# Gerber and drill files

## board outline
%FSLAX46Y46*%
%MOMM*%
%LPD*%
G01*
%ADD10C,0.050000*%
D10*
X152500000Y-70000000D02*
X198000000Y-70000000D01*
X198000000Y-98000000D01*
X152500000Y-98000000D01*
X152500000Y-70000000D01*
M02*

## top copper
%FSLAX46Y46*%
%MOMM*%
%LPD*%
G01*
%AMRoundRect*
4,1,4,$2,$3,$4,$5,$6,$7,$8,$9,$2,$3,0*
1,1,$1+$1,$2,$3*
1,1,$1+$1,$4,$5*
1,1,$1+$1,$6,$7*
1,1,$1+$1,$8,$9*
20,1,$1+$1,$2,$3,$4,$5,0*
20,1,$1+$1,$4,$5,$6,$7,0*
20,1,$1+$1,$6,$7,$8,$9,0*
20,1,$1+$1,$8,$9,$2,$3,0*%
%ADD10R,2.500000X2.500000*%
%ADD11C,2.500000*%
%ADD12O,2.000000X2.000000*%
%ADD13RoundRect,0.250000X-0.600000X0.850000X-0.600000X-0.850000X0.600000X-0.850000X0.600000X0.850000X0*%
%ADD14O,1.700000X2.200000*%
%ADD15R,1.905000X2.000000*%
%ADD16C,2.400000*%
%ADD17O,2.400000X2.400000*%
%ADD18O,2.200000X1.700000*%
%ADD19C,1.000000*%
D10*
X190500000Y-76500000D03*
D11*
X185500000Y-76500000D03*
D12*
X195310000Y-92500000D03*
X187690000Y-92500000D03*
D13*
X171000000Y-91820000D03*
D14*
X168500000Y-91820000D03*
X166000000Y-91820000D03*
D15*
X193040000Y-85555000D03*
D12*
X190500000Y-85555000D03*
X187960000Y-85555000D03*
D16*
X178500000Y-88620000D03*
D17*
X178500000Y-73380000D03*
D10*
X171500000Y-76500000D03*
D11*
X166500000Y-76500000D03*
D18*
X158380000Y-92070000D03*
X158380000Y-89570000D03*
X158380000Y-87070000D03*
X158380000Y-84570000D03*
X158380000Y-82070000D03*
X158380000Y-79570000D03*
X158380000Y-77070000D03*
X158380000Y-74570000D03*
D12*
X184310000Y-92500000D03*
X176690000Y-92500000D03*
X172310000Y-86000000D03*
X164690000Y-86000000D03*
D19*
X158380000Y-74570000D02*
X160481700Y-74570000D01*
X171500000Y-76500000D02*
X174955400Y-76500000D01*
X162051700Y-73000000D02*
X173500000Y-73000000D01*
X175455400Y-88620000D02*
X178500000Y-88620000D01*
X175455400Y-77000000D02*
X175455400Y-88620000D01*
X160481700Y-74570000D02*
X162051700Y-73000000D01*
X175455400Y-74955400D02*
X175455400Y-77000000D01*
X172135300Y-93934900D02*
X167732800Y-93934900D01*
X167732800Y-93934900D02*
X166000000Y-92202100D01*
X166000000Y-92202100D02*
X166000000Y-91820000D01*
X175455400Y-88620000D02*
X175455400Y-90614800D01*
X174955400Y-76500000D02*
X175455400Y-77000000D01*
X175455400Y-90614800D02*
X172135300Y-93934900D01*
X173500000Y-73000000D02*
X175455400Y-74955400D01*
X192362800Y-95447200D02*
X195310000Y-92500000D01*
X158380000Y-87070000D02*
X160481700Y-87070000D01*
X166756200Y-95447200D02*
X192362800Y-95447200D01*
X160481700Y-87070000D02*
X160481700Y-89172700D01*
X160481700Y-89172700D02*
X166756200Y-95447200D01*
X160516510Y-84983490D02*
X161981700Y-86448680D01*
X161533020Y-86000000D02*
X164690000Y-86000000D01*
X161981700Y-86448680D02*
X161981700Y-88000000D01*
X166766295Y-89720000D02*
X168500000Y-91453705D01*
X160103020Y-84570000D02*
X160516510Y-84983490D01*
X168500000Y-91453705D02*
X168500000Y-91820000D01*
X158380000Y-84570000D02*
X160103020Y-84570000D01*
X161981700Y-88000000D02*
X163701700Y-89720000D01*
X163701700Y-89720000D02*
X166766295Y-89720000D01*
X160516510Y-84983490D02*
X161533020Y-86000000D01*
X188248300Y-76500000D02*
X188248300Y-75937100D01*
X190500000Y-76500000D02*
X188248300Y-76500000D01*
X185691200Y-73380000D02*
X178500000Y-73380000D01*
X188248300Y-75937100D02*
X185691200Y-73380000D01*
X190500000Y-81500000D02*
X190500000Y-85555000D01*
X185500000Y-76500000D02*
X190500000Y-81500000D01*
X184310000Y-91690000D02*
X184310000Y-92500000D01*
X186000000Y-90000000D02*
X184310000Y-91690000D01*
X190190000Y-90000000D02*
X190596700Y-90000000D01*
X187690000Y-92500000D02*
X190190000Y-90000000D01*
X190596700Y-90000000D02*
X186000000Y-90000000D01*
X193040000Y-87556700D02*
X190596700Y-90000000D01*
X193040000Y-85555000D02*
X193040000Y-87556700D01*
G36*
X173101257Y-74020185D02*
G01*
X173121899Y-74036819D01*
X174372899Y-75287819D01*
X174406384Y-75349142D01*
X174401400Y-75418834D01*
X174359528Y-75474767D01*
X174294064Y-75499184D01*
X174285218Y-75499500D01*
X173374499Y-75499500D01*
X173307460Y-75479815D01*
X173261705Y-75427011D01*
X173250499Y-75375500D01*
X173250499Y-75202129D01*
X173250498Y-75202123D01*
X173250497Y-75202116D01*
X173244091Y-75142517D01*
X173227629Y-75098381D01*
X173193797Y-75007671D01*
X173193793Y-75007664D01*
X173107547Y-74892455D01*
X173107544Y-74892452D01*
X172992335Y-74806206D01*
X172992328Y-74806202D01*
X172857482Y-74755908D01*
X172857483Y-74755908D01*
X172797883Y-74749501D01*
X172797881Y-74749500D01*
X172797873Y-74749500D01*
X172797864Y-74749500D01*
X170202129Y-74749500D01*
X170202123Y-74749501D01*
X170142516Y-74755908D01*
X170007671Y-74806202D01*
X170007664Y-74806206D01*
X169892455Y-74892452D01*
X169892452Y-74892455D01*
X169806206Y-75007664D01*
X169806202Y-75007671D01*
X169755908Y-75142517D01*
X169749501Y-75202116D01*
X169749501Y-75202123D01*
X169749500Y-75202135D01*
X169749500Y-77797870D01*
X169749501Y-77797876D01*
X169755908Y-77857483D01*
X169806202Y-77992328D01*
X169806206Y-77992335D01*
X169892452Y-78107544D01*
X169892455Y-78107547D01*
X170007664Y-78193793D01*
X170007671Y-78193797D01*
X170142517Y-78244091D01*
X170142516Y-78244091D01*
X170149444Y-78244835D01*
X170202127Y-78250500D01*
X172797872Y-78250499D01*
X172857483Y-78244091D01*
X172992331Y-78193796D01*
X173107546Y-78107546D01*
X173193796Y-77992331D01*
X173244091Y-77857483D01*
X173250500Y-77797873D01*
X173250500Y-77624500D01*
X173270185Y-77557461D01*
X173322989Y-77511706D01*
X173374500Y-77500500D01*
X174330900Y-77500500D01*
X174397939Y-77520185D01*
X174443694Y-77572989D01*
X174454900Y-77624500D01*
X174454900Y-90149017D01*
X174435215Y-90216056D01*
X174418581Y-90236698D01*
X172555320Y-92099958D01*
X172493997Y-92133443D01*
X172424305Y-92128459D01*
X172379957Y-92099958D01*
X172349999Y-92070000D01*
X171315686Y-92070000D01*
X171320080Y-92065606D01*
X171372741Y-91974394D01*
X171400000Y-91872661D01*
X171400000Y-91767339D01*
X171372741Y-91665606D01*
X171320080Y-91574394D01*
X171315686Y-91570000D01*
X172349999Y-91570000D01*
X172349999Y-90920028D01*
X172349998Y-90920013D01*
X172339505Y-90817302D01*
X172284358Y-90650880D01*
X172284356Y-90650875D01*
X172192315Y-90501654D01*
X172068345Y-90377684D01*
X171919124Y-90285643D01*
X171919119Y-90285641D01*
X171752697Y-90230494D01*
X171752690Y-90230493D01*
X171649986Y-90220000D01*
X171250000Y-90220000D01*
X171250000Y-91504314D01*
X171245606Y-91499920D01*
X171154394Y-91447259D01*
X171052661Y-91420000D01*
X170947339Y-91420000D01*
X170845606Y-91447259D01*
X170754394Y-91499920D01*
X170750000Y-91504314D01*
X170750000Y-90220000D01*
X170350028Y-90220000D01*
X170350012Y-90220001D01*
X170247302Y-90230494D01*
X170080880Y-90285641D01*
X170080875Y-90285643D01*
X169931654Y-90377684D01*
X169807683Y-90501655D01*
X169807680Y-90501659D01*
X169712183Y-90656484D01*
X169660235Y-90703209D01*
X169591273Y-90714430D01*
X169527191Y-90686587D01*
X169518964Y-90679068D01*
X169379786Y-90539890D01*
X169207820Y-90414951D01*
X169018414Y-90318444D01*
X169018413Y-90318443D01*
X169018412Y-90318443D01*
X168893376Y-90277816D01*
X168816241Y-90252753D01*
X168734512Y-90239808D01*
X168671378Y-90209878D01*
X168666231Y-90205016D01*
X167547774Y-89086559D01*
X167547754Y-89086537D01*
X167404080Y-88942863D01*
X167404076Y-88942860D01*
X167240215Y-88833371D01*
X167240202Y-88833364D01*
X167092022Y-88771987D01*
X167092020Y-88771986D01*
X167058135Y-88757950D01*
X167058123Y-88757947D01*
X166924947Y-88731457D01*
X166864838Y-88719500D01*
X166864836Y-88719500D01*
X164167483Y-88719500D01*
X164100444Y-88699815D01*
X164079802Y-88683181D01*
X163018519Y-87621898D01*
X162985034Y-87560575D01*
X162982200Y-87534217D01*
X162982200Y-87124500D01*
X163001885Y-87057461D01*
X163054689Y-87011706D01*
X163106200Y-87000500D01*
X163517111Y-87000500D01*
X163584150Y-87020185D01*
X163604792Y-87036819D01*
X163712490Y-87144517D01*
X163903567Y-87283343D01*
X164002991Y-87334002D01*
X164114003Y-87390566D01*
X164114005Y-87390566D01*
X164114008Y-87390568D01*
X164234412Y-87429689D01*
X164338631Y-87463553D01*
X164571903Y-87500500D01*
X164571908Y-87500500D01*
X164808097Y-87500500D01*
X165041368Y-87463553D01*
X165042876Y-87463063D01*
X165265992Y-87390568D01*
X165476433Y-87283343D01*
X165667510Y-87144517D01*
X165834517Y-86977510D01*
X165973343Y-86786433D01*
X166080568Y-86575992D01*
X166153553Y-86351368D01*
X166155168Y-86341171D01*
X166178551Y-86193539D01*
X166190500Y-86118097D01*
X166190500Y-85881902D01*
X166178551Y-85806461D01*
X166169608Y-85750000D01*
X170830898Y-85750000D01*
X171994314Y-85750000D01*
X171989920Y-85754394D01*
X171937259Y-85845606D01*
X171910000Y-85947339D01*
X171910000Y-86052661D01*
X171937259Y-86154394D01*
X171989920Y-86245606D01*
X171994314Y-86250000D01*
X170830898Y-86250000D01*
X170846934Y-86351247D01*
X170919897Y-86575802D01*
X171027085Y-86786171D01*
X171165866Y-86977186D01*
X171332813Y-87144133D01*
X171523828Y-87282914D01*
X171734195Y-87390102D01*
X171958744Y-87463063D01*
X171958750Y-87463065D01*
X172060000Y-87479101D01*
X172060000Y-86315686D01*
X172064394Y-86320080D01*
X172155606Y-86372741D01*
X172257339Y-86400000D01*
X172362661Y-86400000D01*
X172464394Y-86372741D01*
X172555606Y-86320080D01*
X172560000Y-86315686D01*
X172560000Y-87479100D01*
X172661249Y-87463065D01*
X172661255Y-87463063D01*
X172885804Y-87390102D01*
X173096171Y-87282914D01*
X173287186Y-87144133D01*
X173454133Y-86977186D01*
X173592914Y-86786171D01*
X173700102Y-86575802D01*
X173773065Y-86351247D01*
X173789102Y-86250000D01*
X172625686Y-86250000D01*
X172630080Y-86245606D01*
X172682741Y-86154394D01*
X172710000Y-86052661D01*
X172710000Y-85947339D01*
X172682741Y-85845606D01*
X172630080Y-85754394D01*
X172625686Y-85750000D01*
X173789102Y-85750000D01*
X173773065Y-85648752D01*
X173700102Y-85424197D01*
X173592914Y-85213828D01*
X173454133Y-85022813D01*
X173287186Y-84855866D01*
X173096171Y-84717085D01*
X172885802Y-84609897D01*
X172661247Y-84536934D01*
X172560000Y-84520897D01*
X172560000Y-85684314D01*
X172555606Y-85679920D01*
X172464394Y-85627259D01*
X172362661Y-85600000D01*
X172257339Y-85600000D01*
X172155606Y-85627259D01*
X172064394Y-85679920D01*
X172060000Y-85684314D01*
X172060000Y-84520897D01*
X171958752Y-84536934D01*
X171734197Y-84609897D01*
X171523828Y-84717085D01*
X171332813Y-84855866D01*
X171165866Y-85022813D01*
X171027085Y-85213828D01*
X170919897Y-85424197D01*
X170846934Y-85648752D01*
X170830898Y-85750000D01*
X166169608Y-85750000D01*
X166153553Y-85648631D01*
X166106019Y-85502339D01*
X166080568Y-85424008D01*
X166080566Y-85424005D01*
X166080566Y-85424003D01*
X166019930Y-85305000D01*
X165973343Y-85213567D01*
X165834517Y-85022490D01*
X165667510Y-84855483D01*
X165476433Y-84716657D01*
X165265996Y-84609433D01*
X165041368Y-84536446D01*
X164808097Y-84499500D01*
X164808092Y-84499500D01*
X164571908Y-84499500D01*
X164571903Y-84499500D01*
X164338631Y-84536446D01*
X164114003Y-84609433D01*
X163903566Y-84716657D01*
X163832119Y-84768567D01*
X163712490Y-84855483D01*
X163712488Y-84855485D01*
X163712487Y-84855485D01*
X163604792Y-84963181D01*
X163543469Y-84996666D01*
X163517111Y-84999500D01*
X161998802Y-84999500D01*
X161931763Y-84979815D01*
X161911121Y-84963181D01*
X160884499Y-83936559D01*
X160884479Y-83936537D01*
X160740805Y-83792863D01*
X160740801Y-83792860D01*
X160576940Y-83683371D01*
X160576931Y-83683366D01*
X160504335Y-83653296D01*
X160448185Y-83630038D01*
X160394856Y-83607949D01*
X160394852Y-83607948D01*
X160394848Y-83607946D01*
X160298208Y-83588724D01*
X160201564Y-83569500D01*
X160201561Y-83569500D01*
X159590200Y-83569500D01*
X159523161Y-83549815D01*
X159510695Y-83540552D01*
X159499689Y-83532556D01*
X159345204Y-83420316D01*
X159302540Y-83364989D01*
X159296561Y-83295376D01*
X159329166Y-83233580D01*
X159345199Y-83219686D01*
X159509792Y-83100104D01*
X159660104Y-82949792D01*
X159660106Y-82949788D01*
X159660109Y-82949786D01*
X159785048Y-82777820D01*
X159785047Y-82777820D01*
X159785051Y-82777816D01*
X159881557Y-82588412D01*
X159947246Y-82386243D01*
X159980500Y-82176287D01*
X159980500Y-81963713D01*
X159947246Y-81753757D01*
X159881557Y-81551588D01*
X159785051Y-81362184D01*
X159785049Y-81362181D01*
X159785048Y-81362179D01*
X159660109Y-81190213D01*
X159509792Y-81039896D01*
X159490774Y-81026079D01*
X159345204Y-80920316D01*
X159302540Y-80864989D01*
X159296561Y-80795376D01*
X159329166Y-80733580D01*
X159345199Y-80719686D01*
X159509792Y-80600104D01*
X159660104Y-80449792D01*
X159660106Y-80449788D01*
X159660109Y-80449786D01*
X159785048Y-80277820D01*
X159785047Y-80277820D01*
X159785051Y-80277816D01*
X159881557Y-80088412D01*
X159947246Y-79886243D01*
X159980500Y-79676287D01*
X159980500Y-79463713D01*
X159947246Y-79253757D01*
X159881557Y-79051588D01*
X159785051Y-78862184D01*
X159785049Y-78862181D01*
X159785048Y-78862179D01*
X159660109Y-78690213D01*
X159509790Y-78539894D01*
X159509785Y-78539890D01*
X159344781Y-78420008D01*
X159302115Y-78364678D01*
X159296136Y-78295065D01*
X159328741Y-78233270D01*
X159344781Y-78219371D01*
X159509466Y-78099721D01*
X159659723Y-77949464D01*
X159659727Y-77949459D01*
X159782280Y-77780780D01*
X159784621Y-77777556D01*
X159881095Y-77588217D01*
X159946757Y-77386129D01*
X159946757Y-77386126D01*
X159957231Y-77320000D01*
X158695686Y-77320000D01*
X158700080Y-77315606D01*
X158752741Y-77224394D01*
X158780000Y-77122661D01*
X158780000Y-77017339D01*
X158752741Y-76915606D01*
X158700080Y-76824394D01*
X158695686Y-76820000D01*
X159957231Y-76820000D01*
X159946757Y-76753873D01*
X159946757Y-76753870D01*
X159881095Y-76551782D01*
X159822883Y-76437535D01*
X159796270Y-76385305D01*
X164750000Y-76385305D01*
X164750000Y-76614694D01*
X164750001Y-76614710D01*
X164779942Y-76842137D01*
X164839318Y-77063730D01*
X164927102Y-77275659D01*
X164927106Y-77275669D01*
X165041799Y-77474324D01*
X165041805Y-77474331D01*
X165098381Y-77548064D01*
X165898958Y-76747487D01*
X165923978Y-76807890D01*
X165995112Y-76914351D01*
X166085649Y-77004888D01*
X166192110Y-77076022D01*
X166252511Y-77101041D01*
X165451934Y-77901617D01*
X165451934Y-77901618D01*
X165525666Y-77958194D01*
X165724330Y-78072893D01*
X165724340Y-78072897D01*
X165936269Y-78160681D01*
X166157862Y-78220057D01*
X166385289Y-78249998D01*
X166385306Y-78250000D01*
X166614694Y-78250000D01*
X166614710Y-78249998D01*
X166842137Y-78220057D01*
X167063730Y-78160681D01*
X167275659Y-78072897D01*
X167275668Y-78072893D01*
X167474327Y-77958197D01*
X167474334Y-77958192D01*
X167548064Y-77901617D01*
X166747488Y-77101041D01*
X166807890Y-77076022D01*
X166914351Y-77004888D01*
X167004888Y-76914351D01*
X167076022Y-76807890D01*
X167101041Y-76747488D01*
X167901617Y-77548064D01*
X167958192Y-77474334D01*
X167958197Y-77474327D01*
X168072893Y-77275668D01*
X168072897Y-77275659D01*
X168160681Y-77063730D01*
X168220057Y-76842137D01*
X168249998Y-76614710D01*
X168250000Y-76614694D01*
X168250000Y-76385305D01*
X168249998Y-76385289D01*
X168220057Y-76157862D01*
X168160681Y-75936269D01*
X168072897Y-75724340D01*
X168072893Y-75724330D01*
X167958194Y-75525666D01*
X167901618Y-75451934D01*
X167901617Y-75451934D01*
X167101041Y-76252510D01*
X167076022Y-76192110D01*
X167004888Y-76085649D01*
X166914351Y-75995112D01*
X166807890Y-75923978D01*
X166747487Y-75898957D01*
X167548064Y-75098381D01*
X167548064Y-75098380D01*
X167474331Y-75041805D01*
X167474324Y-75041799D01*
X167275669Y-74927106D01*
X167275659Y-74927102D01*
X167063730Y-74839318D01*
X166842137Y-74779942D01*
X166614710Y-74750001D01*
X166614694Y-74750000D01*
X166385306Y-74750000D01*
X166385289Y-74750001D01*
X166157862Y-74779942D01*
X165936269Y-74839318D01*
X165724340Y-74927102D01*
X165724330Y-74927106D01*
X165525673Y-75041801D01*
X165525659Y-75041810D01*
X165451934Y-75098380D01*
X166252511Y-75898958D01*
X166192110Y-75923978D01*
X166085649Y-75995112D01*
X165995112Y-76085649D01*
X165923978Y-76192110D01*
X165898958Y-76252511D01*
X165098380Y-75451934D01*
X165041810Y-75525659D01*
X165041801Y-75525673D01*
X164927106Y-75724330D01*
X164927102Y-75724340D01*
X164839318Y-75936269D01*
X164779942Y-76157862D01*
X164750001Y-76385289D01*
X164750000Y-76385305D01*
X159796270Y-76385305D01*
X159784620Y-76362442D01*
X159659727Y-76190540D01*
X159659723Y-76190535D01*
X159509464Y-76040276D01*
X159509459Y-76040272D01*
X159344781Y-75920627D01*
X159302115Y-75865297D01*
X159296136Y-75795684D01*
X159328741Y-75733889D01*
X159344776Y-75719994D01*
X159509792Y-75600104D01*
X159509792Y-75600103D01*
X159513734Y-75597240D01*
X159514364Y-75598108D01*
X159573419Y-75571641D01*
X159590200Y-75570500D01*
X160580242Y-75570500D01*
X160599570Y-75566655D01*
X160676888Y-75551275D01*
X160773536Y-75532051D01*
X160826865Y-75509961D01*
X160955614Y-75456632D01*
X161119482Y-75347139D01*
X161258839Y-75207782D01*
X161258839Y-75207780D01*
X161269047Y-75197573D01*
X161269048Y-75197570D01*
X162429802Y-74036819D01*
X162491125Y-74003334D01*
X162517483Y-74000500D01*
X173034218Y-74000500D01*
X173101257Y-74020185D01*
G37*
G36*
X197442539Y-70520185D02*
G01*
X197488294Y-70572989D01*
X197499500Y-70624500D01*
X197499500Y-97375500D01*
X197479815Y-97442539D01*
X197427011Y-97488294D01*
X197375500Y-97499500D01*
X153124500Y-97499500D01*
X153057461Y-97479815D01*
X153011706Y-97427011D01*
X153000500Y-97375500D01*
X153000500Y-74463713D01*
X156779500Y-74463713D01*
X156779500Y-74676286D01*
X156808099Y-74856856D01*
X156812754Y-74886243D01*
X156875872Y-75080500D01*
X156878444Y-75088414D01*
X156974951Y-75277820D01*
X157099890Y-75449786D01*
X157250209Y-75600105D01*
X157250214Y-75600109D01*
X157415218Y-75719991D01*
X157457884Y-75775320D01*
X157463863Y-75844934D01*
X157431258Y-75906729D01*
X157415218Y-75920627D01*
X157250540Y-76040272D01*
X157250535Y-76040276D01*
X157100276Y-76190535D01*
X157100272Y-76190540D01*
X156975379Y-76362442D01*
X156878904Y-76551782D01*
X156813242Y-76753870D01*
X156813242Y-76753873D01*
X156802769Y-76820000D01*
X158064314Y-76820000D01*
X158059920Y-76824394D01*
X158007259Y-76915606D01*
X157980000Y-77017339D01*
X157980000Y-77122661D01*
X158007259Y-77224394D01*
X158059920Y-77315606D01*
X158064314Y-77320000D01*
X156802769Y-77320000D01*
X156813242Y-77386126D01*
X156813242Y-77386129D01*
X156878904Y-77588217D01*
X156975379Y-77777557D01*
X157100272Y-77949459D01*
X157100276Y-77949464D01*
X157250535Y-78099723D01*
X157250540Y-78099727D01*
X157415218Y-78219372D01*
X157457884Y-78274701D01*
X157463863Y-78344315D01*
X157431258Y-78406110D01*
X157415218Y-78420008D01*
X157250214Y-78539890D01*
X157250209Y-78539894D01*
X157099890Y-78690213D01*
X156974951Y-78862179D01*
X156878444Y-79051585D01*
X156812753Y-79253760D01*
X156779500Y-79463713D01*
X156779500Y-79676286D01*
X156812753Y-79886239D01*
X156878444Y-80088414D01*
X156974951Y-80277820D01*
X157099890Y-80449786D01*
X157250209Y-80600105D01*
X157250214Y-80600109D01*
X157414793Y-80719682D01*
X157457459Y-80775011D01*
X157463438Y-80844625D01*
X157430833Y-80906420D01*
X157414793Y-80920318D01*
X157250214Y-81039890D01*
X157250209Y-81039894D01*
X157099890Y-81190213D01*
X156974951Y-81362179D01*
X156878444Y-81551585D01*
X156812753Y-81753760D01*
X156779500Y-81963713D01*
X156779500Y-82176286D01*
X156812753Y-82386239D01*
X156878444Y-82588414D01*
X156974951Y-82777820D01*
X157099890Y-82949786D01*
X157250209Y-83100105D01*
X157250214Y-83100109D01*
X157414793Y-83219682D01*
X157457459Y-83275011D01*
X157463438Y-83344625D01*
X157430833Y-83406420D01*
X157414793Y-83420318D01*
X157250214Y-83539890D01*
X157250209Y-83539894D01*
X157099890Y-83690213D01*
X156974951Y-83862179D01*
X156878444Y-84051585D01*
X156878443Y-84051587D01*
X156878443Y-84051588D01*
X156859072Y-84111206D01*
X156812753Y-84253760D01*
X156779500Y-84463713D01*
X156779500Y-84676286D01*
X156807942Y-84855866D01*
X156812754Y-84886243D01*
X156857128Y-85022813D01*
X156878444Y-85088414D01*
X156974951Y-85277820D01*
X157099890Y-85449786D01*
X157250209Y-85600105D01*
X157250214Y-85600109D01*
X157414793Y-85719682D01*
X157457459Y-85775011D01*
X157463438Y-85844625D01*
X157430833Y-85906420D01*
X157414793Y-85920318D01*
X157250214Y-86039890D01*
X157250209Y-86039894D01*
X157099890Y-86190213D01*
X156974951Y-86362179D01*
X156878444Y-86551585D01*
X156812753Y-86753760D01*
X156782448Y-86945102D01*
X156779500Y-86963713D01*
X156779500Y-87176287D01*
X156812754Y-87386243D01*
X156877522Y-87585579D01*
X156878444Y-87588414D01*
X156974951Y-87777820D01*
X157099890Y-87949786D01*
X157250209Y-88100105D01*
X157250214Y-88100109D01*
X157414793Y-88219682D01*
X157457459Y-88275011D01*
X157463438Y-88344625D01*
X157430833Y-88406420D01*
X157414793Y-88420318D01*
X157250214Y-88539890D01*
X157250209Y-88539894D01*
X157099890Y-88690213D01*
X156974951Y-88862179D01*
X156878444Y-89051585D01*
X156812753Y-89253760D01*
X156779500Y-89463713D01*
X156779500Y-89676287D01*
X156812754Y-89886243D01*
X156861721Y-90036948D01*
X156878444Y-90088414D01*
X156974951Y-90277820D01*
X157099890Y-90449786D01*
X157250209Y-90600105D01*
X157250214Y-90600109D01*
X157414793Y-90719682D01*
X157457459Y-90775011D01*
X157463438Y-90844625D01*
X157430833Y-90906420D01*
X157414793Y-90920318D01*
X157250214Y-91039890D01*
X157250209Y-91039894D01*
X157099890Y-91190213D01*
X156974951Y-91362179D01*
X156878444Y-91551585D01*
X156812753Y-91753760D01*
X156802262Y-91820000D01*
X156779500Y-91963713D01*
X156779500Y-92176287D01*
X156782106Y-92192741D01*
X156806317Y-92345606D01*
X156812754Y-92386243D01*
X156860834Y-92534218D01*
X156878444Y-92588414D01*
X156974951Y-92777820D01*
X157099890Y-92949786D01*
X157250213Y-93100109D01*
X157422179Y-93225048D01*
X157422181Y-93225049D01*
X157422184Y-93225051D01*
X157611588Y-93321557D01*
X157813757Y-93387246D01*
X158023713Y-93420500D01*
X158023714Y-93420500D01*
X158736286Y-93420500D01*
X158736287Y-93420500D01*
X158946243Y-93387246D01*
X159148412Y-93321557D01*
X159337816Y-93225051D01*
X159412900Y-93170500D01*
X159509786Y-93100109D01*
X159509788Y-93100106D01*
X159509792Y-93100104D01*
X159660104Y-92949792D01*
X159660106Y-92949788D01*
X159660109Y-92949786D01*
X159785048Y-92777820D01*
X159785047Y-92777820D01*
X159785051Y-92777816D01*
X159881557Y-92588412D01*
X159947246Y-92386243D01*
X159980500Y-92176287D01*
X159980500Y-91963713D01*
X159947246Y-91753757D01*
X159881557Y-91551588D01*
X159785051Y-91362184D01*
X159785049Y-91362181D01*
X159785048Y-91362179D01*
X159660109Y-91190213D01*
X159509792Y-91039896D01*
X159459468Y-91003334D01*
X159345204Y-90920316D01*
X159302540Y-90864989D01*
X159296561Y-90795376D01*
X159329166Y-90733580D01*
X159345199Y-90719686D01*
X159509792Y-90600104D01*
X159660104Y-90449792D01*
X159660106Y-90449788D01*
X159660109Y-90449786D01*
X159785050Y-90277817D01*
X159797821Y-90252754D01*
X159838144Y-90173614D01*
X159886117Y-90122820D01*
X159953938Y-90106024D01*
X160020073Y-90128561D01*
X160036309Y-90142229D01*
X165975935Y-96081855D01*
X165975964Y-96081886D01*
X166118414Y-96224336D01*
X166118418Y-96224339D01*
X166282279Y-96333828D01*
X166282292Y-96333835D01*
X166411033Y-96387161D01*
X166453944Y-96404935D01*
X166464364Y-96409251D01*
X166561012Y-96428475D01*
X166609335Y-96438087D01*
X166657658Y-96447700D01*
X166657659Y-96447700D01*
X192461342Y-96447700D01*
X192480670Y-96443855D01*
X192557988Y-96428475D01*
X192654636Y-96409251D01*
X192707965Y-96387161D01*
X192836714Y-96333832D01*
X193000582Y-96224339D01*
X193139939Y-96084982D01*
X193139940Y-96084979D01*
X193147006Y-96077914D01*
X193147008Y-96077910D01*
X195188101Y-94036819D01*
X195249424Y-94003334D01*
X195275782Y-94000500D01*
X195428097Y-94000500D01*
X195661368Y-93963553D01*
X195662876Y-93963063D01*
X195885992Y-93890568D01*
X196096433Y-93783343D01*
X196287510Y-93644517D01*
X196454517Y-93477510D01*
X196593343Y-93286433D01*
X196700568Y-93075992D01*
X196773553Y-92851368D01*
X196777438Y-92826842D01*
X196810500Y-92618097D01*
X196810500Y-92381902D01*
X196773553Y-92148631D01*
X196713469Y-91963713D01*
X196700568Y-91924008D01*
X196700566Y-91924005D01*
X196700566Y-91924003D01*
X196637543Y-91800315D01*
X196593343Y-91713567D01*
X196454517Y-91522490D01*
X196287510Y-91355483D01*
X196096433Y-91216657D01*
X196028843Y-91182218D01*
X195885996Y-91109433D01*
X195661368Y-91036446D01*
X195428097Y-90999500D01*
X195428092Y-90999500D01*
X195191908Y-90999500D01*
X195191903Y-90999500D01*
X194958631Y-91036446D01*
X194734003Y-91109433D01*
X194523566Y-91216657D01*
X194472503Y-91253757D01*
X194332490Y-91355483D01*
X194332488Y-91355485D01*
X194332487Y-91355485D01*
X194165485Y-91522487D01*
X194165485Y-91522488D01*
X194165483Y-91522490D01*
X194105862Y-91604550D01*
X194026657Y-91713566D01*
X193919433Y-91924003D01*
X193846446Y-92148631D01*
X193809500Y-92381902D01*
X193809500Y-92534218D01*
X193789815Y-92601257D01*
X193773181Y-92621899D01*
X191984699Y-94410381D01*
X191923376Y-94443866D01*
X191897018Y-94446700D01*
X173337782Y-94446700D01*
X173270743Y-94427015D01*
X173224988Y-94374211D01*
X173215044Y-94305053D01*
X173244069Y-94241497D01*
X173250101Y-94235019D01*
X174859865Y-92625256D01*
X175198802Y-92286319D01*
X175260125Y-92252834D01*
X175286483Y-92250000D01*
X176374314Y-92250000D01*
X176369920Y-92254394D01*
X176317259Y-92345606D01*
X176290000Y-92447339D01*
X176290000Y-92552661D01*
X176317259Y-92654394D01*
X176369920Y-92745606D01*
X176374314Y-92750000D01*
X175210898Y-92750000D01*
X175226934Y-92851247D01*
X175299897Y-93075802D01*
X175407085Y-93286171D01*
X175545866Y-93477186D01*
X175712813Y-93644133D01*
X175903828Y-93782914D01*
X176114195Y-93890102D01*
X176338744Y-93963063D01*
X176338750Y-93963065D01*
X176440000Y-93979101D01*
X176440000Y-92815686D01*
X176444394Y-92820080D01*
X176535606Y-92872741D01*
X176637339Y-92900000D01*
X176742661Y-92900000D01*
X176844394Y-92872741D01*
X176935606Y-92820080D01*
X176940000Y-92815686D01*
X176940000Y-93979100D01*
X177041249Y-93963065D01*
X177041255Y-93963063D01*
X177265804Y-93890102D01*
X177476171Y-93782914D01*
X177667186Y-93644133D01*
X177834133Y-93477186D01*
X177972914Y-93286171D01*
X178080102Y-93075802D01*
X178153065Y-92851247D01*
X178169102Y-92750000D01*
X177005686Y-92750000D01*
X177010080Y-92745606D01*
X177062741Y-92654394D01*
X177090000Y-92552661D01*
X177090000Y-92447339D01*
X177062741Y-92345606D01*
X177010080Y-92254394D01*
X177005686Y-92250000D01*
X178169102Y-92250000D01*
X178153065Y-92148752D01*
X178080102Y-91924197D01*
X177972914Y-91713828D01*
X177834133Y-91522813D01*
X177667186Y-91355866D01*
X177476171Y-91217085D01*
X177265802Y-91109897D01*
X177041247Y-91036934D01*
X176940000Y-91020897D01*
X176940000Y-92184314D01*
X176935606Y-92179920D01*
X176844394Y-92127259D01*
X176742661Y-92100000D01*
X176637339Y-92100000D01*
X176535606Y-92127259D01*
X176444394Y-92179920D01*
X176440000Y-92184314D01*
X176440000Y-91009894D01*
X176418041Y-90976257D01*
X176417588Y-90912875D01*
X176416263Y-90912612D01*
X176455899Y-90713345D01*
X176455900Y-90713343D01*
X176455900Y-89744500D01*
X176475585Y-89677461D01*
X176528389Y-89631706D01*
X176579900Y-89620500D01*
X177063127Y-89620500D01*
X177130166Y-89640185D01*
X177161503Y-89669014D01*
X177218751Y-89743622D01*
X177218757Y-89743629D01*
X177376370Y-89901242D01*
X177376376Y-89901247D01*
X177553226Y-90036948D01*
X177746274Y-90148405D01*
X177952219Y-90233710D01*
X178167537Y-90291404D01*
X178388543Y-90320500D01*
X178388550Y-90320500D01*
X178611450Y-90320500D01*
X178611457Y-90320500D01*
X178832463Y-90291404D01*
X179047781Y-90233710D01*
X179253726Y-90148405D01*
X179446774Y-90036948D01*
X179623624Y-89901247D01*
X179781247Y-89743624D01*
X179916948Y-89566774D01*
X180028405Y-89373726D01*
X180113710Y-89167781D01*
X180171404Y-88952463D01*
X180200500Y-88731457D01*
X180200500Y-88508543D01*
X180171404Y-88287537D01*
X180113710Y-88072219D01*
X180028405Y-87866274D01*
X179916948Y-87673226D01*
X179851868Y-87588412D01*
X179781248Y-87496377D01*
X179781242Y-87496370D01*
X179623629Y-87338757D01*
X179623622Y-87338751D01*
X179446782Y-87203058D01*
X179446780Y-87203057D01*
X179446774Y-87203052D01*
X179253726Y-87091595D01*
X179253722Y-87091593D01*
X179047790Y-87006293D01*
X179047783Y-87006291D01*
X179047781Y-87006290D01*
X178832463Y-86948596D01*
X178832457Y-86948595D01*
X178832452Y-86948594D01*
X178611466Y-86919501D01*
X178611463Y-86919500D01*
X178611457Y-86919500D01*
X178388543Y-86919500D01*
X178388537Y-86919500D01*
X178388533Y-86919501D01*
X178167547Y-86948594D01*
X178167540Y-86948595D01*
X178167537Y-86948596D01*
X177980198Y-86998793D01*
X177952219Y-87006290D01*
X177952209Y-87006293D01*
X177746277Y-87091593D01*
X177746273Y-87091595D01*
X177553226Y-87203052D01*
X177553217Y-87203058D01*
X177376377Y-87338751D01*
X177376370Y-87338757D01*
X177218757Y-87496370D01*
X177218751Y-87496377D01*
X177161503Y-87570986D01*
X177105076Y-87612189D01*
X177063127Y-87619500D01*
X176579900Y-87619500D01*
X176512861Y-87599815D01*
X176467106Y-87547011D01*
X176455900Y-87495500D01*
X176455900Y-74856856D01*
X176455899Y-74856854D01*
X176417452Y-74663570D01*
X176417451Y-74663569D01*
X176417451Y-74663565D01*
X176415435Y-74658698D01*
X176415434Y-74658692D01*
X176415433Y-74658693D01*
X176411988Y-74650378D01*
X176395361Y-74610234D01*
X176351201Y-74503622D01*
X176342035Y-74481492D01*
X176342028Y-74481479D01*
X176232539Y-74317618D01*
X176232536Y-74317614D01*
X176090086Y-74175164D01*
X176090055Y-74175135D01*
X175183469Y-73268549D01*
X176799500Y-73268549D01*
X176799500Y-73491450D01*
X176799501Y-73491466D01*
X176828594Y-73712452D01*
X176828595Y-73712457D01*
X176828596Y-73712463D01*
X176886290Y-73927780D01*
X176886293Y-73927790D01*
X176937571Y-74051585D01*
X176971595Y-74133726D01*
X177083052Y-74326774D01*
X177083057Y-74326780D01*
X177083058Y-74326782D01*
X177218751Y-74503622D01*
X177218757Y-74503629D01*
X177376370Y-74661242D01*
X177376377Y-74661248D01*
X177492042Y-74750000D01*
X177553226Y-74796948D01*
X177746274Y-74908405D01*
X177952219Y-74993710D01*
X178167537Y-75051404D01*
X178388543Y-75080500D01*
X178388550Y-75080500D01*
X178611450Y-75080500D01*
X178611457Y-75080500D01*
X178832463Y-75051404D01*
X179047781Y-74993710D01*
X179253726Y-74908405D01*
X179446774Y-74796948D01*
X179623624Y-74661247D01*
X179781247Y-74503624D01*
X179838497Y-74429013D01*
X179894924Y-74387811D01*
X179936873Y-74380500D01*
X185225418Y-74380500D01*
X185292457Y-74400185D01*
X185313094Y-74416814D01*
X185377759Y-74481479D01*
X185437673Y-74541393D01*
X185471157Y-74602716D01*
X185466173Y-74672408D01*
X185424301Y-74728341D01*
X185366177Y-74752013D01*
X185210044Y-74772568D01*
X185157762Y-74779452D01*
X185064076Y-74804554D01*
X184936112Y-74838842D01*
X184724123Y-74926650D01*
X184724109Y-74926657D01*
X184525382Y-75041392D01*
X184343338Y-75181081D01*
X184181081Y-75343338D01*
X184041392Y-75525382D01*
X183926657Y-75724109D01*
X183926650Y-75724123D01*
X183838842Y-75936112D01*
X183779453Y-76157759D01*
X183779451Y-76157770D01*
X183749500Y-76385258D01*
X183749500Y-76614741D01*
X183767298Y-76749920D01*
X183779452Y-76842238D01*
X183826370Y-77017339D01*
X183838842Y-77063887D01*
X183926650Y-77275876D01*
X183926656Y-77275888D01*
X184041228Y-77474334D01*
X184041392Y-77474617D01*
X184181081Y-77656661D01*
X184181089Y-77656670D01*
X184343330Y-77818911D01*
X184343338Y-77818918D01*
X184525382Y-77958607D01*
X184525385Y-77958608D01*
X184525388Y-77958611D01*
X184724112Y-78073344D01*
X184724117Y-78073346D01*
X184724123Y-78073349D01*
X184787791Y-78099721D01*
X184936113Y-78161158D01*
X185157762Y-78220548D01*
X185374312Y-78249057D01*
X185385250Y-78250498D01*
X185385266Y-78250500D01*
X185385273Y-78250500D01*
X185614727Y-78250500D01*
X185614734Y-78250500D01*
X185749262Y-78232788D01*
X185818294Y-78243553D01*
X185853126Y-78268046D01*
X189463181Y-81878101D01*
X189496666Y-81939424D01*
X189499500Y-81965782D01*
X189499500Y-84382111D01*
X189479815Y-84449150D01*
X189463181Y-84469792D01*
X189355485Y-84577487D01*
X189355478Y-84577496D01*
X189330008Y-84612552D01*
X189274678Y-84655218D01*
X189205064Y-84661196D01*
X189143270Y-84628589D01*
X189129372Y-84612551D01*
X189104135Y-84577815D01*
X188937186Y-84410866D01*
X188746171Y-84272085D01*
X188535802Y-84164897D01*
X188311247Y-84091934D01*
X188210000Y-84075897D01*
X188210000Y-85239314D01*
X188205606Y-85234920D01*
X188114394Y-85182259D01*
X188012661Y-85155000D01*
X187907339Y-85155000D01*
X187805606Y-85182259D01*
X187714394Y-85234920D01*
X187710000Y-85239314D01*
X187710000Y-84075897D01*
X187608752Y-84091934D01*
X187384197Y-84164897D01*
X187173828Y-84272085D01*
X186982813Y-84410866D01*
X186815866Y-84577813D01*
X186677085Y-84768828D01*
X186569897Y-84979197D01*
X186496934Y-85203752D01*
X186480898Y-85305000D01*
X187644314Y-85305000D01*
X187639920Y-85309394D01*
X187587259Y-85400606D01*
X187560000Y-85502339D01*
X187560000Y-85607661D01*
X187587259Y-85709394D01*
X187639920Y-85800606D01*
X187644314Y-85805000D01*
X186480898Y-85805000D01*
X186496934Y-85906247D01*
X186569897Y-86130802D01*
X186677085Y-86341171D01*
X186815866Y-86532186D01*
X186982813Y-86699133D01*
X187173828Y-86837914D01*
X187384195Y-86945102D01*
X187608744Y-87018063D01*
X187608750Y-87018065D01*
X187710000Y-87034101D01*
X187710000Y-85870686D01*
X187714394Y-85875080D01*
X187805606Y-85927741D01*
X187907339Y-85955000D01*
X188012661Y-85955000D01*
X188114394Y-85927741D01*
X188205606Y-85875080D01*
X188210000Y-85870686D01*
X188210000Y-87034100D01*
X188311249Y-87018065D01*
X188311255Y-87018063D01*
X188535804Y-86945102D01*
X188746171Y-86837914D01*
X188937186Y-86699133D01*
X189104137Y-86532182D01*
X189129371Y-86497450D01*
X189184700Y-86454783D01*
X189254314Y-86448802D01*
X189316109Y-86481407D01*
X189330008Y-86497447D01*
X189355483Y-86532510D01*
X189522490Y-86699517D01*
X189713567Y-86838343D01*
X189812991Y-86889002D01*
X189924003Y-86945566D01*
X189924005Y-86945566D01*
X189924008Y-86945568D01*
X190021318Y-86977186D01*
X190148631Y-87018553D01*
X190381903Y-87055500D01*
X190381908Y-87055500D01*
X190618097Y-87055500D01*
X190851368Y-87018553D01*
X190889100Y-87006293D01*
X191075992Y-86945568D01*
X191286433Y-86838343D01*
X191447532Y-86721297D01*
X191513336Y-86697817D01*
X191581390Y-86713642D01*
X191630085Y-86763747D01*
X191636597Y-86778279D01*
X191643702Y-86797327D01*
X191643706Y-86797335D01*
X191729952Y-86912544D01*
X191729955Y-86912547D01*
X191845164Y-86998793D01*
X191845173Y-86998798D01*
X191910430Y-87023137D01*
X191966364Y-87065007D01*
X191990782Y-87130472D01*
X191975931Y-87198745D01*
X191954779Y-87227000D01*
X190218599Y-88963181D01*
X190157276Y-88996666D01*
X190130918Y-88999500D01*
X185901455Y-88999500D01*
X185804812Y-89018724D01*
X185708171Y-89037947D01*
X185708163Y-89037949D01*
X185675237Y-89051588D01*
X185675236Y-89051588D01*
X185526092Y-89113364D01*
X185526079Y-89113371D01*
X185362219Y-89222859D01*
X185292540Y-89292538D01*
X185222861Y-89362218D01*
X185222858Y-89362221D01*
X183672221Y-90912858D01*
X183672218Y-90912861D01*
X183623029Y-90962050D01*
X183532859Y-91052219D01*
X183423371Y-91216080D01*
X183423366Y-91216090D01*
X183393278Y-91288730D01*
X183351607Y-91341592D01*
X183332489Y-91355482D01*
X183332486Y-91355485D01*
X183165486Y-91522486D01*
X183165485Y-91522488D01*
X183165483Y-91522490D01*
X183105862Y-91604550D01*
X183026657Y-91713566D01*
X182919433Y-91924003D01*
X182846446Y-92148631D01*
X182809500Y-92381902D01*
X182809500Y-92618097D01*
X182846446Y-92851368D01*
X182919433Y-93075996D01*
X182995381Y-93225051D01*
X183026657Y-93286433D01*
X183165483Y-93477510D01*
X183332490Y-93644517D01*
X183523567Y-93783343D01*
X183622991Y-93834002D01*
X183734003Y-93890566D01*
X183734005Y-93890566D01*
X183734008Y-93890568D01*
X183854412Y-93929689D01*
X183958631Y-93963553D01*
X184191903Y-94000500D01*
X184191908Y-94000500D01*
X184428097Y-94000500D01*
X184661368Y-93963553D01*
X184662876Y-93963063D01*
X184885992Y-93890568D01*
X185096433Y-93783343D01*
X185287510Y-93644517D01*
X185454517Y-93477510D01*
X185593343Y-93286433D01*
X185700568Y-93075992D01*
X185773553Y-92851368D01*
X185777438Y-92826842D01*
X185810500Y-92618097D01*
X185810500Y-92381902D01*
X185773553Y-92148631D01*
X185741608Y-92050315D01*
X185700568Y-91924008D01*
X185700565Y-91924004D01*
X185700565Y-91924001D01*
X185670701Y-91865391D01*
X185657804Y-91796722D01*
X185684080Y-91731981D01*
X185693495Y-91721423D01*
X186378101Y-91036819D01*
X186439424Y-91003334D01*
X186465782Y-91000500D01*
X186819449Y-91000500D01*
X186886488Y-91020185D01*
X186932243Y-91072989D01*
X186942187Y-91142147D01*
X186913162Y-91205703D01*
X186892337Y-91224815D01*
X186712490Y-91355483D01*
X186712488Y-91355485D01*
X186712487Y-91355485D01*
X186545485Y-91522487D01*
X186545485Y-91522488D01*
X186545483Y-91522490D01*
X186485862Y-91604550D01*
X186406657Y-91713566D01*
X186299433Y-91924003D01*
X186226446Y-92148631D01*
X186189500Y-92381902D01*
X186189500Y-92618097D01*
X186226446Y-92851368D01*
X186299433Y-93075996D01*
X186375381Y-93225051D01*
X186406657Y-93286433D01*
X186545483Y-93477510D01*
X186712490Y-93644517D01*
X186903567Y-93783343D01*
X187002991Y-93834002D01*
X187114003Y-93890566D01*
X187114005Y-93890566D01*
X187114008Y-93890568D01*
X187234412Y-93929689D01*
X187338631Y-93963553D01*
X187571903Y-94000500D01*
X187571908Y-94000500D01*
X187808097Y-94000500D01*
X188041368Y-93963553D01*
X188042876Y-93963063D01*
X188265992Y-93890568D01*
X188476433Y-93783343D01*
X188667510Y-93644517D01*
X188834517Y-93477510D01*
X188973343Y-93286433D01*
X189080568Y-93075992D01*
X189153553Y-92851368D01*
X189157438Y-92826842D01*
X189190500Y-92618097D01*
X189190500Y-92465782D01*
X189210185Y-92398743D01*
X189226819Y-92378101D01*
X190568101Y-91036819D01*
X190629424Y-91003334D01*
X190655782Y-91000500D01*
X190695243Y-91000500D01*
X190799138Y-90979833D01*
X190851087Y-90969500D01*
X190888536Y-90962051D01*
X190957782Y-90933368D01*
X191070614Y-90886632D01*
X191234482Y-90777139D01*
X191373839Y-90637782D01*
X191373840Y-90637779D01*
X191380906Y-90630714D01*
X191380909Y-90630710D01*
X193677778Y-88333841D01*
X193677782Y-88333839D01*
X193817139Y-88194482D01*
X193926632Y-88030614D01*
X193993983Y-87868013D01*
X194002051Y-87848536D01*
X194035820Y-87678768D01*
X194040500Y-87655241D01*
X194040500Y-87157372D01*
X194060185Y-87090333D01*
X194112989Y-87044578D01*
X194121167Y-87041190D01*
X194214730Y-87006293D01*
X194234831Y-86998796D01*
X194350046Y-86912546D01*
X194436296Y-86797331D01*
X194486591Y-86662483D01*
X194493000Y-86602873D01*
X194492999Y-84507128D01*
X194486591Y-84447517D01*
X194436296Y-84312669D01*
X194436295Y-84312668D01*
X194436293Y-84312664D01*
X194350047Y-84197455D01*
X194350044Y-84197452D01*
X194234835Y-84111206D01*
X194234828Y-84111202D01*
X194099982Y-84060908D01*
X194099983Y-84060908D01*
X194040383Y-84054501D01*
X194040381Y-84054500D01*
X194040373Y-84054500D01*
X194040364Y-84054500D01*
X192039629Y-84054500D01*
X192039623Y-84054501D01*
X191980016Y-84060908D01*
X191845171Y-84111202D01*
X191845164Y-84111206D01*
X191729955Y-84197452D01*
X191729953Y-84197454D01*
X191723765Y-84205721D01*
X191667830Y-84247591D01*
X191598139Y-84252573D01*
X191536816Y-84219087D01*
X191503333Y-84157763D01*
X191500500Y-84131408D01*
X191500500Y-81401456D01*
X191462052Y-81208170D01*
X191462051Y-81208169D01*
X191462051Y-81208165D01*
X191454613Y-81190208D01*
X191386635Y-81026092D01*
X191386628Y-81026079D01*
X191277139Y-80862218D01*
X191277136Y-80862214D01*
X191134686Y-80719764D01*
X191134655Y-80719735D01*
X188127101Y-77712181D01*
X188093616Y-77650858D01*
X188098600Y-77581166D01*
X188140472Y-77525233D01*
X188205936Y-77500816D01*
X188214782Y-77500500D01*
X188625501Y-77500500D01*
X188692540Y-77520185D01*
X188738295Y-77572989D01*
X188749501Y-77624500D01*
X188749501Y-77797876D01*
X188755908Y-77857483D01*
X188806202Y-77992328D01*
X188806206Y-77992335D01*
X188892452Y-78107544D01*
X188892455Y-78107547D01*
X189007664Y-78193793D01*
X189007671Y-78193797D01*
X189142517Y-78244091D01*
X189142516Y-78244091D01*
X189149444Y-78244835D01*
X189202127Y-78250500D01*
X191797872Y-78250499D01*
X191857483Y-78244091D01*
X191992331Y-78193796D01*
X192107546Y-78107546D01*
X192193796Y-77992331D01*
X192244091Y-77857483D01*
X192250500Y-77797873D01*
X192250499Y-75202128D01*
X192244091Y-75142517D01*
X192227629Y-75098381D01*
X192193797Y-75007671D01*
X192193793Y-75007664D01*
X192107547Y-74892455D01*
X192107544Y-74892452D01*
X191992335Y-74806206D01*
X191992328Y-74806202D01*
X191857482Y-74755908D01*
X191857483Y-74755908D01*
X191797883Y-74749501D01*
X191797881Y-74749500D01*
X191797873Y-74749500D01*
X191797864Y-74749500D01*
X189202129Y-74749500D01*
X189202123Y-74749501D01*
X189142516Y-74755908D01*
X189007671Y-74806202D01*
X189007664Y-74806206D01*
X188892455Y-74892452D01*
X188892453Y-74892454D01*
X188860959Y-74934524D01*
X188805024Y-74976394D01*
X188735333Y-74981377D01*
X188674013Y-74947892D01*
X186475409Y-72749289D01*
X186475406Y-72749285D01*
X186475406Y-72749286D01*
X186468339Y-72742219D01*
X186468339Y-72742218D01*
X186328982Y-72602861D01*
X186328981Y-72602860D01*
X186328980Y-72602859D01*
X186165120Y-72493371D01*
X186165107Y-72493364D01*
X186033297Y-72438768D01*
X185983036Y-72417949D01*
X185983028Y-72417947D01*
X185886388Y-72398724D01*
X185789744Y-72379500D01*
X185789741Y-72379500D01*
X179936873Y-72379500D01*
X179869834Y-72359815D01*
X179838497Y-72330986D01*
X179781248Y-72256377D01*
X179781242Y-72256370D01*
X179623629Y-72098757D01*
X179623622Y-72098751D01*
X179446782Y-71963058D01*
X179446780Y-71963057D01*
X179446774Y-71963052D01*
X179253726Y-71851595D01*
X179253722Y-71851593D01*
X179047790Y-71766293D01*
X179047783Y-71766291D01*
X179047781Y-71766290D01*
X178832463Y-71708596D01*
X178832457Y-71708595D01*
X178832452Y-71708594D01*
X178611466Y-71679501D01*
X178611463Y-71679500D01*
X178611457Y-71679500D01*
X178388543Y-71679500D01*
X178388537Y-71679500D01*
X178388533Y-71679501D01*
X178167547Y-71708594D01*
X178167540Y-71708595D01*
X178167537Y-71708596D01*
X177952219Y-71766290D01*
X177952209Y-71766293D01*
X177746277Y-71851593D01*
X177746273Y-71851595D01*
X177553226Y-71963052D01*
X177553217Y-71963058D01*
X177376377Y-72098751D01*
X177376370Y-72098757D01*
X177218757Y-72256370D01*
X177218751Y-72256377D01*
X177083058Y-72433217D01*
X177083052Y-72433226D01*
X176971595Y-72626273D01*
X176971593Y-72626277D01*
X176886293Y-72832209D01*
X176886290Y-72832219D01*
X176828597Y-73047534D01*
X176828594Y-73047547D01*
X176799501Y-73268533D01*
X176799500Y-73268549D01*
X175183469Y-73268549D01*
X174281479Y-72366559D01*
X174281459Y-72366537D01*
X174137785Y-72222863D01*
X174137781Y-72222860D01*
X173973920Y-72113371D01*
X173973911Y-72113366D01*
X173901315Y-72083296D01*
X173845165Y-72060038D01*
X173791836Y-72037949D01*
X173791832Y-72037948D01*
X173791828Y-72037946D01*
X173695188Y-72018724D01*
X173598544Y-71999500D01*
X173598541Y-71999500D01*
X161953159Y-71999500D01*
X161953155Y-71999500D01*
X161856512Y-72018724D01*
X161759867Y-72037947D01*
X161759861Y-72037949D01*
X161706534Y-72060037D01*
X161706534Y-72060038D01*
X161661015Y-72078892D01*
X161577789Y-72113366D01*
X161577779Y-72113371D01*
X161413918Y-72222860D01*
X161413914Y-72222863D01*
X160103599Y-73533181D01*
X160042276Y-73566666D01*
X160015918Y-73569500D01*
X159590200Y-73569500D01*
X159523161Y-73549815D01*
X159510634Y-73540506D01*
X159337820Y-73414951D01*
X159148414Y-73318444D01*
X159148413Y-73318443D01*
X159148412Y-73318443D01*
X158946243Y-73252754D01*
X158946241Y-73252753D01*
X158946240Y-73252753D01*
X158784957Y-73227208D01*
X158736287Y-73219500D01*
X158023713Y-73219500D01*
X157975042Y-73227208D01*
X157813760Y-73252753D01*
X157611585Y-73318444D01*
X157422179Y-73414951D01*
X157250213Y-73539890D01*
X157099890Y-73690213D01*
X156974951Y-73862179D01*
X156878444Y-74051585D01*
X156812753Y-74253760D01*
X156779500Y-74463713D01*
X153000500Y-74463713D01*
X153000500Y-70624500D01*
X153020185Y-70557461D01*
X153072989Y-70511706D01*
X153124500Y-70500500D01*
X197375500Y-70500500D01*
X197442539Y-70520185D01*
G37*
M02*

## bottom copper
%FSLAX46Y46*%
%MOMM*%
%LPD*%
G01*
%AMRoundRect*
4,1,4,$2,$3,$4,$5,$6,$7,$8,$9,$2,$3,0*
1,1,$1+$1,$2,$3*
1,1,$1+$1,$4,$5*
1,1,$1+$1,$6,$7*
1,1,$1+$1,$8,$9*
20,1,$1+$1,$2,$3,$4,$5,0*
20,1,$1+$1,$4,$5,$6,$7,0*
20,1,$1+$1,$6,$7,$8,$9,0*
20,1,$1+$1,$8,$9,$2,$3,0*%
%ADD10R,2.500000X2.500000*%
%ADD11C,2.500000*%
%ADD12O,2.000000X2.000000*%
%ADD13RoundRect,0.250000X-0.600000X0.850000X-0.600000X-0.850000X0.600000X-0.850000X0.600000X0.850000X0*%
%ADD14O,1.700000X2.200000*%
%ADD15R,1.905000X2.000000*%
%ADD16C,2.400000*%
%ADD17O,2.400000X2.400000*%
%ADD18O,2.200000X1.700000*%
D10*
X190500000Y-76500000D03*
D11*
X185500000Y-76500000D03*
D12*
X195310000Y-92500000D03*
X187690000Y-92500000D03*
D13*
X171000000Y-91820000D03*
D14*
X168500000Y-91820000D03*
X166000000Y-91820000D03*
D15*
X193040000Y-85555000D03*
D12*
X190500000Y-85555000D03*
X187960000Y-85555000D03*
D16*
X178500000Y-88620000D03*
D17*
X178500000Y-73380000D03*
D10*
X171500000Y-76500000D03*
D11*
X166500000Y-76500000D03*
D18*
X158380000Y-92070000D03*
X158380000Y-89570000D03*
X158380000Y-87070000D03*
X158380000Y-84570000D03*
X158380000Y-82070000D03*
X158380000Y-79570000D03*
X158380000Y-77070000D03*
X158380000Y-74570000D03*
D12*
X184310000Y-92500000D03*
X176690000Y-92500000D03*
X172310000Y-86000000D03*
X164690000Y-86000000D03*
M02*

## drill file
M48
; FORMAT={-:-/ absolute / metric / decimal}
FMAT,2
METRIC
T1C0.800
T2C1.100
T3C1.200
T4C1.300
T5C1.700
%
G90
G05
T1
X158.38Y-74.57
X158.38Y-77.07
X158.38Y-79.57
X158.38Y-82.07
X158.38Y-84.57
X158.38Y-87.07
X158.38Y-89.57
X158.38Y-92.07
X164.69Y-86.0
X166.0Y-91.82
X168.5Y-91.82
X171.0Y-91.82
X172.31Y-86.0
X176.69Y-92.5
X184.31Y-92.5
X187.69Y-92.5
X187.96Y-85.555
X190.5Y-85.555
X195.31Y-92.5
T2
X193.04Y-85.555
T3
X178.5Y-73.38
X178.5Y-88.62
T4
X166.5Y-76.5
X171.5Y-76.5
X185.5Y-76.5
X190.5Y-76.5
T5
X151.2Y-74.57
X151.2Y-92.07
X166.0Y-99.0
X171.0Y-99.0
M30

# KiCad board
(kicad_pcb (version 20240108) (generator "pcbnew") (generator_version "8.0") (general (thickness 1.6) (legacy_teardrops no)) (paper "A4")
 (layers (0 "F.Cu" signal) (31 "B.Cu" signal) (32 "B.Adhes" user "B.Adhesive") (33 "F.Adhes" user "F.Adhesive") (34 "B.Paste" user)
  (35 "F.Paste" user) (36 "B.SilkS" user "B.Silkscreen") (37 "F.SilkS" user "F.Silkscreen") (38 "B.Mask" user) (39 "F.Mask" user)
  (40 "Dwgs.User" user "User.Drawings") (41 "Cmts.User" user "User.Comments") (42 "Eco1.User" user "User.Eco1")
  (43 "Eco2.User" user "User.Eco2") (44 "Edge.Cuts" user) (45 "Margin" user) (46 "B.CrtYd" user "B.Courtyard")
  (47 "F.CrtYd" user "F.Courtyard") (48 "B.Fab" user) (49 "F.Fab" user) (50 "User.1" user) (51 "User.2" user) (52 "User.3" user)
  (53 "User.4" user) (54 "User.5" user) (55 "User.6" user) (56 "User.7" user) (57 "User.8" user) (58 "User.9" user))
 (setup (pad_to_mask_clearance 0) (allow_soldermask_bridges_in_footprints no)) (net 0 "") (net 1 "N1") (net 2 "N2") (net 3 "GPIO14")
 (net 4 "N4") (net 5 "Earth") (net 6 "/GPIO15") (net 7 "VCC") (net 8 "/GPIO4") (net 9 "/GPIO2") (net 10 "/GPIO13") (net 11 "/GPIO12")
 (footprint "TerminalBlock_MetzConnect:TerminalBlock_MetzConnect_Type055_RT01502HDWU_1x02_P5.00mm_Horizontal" (layer "F.Cu")
  (at 190.5 76.5 180)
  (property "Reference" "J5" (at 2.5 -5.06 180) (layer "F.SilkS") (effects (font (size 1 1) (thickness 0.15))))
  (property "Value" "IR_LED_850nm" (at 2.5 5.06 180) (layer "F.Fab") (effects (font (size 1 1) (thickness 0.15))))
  (pad "1" thru_hole rect (at 0 0 180) (size 2.5 2.5) (drill 1.3) (layers "*.Cu" "*.Mask") (remove_unused_layers no) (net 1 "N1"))
  (pad "2" thru_hole circle (at 5 0 180) (size 2.5 2.5) (drill 1.3) (layers "*.Cu" "*.Mask") (remove_unused_layers no) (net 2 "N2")))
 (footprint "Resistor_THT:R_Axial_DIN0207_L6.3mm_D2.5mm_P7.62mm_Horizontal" (layer "F.Cu") (at 195.31 92.5 180)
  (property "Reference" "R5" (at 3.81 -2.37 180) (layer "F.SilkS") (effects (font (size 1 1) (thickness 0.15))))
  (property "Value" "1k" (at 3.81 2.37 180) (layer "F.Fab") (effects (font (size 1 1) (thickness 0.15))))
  (pad "1" thru_hole oval (at 0 0 180) (size 2 2) (drill 0.8) (layers "*.Cu" "*.Mask") (remove_unused_layers no) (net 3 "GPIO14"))
  (pad "2" thru_hole oval (at 7.62 0 180) (size 2 2) (drill 0.8) (layers "*.Cu" "*.Mask") (remove_unused_layers no) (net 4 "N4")))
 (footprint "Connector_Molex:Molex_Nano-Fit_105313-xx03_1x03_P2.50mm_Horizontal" (layer "F.Cu") (at 171 91.82 -90)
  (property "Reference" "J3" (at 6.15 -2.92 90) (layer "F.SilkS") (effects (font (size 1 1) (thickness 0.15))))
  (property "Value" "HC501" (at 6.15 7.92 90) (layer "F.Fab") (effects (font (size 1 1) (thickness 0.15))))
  (pad "" np_thru_hole circle (at 7.18 0 270) (size 1.7 1.7) (drill 1.7) (layers "*.Cu" "*.Mask"))
  (pad "" np_thru_hole circle (at 7.18 5 270) (size 1.7 1.7) (drill 1.7) (layers "*.Cu" "*.Mask"))
  (pad "1" thru_hole roundrect (at 0 0 270) (size 2.2 1.7) (drill 0.8) (layers "*.Cu" "*.Mask") (remove_unused_layers no)
   (roundrect_rratio 0.147059) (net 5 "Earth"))
  (pad "2" thru_hole oval (at 0 2.5 270) (size 2.2 1.7) (drill 0.8) (layers "*.Cu" "*.Mask") (remove_unused_layers no) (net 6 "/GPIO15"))
  (pad "3" thru_hole oval (at 0 5 270) (size 2.2 1.7) (drill 0.8) (layers "*.Cu" "*.Mask") (remove_unused_layers no) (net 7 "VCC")))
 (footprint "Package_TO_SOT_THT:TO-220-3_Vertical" (layer "F.Cu") (at 193.04 85.555 180)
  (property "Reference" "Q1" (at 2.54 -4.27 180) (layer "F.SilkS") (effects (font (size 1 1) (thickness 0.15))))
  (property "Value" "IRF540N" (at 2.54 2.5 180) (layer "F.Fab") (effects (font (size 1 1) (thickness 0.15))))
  (pad "1" thru_hole rect (at 0 0 180) (size 1.905 2) (drill 1.1) (layers "*.Cu" "*.Mask") (remove_unused_layers no) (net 4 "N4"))
  (pad "2" thru_hole oval (at 2.54 0 180) (size 2 2) (drill 0.8) (layers "*.Cu" "*.Mask") (remove_unused_layers no) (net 2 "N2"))
  (pad "3" thru_hole oval (at 5.08 0 180) (size 2 2) (drill 0.8) (layers "*.Cu" "*.Mask") (remove_unused_layers no) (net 5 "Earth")))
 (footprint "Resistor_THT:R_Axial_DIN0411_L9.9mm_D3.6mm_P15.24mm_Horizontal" (layer "F.Cu") (at 178.5 88.62 90)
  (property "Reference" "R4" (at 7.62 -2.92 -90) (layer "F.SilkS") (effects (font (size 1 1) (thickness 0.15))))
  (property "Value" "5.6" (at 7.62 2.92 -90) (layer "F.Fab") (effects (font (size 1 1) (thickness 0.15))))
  (pad "1" thru_hole circle (at 0 0 90) (size 2.4 2.4) (drill 1.2) (layers "*.Cu" "*.Mask") (remove_unused_layers no) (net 7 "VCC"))
  (pad "2" thru_hole oval (at 15.24 0 90) (size 2.4 2.4) (drill 1.2) (layers "*.Cu" "*.Mask") (remove_unused_layers no) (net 1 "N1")))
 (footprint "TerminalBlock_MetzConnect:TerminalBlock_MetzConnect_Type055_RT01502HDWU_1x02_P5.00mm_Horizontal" (layer "F.Cu")
  (at 171.5 76.5 180)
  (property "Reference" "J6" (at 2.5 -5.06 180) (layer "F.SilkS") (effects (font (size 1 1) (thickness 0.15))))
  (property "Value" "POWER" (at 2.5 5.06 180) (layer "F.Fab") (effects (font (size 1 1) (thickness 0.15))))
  (pad "1" thru_hole rect (at 0 0 180) (size 2.5 2.5) (drill 1.3) (layers "*.Cu" "*.Mask") (remove_unused_layers no) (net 7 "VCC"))
  (pad "2" thru_hole circle (at 5 0 180) (size 2.5 2.5) (drill 1.3) (layers "*.Cu" "*.Mask") (remove_unused_layers no) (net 5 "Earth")))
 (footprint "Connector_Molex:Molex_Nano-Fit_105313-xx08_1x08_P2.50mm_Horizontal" (layer "F.Cu") (at 158.38 92.07 180)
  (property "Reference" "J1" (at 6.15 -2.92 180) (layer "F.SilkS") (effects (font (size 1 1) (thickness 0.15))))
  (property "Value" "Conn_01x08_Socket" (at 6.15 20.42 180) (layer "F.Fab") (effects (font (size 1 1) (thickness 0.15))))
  (pad "" np_thru_hole circle (at 7.18 0 180) (size 1.7 1.7) (drill 1.7) (layers "*.Cu" "*.Mask"))
  (pad "" np_thru_hole circle (at 7.18 17.5 180) (size 1.7 1.7) (drill 1.7) (layers "*.Cu" "*.Mask"))
  (pad "1" thru_hole oval (at 0 0 180) (size 2.2 1.7) (drill 0.8) (layers "*.Cu" "*.Mask") (remove_unused_layers no) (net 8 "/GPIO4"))
  (pad "2" thru_hole oval (at 0 2.5 180) (size 2.2 1.7) (drill 0.8) (layers "*.Cu" "*.Mask") (remove_unused_layers no) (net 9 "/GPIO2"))
  (pad "3" thru_hole oval (at 0 5 180) (size 2.2 1.7) (drill 0.8) (layers "*.Cu" "*.Mask") (remove_unused_layers no) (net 3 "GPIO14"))
  (pad "4" thru_hole oval (at 0 7.5 180) (size 2.2 1.7) (drill 0.8) (layers "*.Cu" "*.Mask") (remove_unused_layers no) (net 6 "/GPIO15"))
  (pad "5" thru_hole oval (at 0 10 180) (size 2.2 1.7) (drill 0.8) (layers "*.Cu" "*.Mask") (remove_unused_layers no) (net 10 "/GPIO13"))
  (pad "6" thru_hole oval (at 0 12.5 180) (size 2.2 1.7) (drill 0.8) (layers "*.Cu" "*.Mask") (remove_unused_layers no) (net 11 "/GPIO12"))
  (pad "7" thru_hole oval (at 0 15 180) (size 2.2 1.7) (drill 0.8) (layers "*.Cu" "*.Mask") (remove_unused_layers no) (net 5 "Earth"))
  (pad "8" thru_hole oval (at 0 17.5 180) (size 2.2 1.7) (drill 0.8) (layers "*.Cu" "*.Mask") (remove_unused_layers no) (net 7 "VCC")))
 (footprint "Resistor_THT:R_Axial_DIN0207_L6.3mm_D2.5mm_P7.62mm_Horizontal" (layer "F.Cu") (at 184.31 92.5 180)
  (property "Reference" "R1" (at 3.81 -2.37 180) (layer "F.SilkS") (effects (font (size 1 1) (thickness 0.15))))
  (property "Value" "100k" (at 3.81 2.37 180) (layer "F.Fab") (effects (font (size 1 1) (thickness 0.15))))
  (pad "1" thru_hole oval (at 0 0 180) (size 2 2) (drill 0.8) (layers "*.Cu" "*.Mask") (remove_unused_layers no) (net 4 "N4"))
  (pad "2" thru_hole oval (at 7.62 0 180) (size 2 2) (drill 0.8) (layers "*.Cu" "*.Mask") (remove_unused_layers no) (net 5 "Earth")))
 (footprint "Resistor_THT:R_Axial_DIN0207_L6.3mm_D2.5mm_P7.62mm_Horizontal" (layer "F.Cu") (at 172.31 86 180)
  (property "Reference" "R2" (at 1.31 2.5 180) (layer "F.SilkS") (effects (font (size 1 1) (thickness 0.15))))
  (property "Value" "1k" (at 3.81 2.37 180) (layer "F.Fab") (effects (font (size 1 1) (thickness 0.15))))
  (pad "1" thru_hole oval (at 0 0 180) (size 2 2) (drill 0.8) (layers "*.Cu" "*.Mask") (remove_unused_layers no) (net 5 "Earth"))
  (pad "2" thru_hole oval (at 7.62 0 180) (size 2 2) (drill 0.8) (layers "*.Cu" "*.Mask") (remove_unused_layers no) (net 6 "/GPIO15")))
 (gr_rect (start 152.5 70) (end 198 98) (stroke (width 0.05) (type default)) (fill none) (layer "Edge.Cuts"))
 (segment (start 158.38 74.57) (end 160.4817 74.57) (width 1) (layer "F.Cu") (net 7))
 (segment (start 171.5 76.5) (end 174.9554 76.5) (width 1) (layer "F.Cu") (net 7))
 (segment (start 162.0517 73) (end 173.5 73) (width 1) (layer "F.Cu") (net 7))
 (segment (start 175.4554 88.62) (end 178.5 88.62) (width 1) (layer "F.Cu") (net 7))
 (segment (start 175.4554 77) (end 175.4554 88.62) (width 1) (layer "F.Cu") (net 7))
 (segment (start 160.4817 74.57) (end 162.0517 73) (width 1) (layer "F.Cu") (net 7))
 (segment (start 175.4554 74.9554) (end 175.4554 77) (width 1) (layer "F.Cu") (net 7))
 (segment (start 172.1353 93.9349) (end 167.7328 93.9349) (width 1) (layer "F.Cu") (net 7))
 (segment (start 167.7328 93.9349) (end 166 92.2021) (width 1) (layer "F.Cu") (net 7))
 (segment (start 166 92.2021) (end 166 91.82) (width 1) (layer "F.Cu") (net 7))
 (segment (start 175.4554 88.62) (end 175.4554 90.6148) (width 1) (layer "F.Cu") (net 7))
 (segment (start 174.9554 76.5) (end 175.4554 77) (width 1) (layer "F.Cu") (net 7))
 (segment (start 175.4554 90.6148) (end 172.1353 93.9349) (width 1) (layer "F.Cu") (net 7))
 (segment (start 173.5 73) (end 175.4554 74.9554) (width 1) (layer "F.Cu") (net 7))
 (segment (start 192.3628 95.4472) (end 195.31 92.5) (width 1) (layer "F.Cu") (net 3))
 (segment (start 158.38 87.07) (end 160.4817 87.07) (width 1) (layer "F.Cu") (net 3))
 (segment (start 166.7562 95.4472) (end 192.3628 95.4472) (width 1) (layer "F.Cu") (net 3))
 (segment (start 160.4817 87.07) (end 160.4817 89.1727) (width 1) (layer "F.Cu") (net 3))
 (segment (start 160.4817 89.1727) (end 166.7562 95.4472) (width 1) (layer "F.Cu") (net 3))
 (segment (start 160.51651 84.98349) (end 161.9817 86.44868) (width 1) (layer "F.Cu") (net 6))
 (segment (start 161.53302 86) (end 164.69 86) (width 1) (layer "F.Cu") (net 6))
 (segment (start 161.9817 86.44868) (end 161.9817 88) (width 1) (layer "F.Cu") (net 6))
 (segment (start 166.766295 89.72) (end 168.5 91.453705) (width 1) (layer "F.Cu") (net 6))
 (segment (start 160.10302 84.57) (end 160.51651 84.98349) (width 1) (layer "F.Cu") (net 6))
 (segment (start 168.5 91.453705) (end 168.5 91.82) (width 1) (layer "F.Cu") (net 6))
 (segment (start 158.38 84.57) (end 160.10302 84.57) (width 1) (layer "F.Cu") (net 6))
 (segment (start 161.9817 88) (end 163.7017 89.72) (width 1) (layer "F.Cu") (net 6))
 (segment (start 163.7017 89.72) (end 166.766295 89.72) (width 1) (layer "F.Cu") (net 6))
 (segment (start 160.51651 84.98349) (end 161.53302 86) (width 1) (layer "F.Cu") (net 6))
 (segment (start 188.2483 76.5) (end 188.2483 75.9371) (width 1) (layer "F.Cu") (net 1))
 (segment (start 190.5 76.5) (end 188.2483 76.5) (width 1) (layer "F.Cu") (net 1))
 (segment (start 185.6912 73.38) (end 178.5 73.38) (width 1) (layer "F.Cu") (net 1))
 (segment (start 188.2483 75.9371) (end 185.6912 73.38) (width 1) (layer "F.Cu") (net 1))
 (segment (start 190.5 81.5) (end 190.5 85.555) (width 1) (layer "F.Cu") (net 2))
 (segment (start 185.5 76.5) (end 190.5 81.5) (width 1) (layer "F.Cu") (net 2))
 (segment (start 184.31 91.69) (end 184.31 92.5) (width 1) (layer "F.Cu") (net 4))
 (segment (start 186 90) (end 184.31 91.69) (width 1) (layer "F.Cu") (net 4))
 (segment (start 190.19 90) (end 190.5967 90) (width 1) (layer "F.Cu") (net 4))
 (segment (start 187.69 92.5) (end 190.19 90) (width 1) (layer "F.Cu") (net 4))
 (segment (start 190.5967 90) (end 186 90) (width 1) (layer "F.Cu") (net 4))
 (segment (start 193.04 87.5567) (end 190.5967 90) (width 1) (layer "F.Cu") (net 4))
 (segment (start 193.04 85.555) (end 193.04 87.5567) (width 1) (layer "F.Cu") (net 4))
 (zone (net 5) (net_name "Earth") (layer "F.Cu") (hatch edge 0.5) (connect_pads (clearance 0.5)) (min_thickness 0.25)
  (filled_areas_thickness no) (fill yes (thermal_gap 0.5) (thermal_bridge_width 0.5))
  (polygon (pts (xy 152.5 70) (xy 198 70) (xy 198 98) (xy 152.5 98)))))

